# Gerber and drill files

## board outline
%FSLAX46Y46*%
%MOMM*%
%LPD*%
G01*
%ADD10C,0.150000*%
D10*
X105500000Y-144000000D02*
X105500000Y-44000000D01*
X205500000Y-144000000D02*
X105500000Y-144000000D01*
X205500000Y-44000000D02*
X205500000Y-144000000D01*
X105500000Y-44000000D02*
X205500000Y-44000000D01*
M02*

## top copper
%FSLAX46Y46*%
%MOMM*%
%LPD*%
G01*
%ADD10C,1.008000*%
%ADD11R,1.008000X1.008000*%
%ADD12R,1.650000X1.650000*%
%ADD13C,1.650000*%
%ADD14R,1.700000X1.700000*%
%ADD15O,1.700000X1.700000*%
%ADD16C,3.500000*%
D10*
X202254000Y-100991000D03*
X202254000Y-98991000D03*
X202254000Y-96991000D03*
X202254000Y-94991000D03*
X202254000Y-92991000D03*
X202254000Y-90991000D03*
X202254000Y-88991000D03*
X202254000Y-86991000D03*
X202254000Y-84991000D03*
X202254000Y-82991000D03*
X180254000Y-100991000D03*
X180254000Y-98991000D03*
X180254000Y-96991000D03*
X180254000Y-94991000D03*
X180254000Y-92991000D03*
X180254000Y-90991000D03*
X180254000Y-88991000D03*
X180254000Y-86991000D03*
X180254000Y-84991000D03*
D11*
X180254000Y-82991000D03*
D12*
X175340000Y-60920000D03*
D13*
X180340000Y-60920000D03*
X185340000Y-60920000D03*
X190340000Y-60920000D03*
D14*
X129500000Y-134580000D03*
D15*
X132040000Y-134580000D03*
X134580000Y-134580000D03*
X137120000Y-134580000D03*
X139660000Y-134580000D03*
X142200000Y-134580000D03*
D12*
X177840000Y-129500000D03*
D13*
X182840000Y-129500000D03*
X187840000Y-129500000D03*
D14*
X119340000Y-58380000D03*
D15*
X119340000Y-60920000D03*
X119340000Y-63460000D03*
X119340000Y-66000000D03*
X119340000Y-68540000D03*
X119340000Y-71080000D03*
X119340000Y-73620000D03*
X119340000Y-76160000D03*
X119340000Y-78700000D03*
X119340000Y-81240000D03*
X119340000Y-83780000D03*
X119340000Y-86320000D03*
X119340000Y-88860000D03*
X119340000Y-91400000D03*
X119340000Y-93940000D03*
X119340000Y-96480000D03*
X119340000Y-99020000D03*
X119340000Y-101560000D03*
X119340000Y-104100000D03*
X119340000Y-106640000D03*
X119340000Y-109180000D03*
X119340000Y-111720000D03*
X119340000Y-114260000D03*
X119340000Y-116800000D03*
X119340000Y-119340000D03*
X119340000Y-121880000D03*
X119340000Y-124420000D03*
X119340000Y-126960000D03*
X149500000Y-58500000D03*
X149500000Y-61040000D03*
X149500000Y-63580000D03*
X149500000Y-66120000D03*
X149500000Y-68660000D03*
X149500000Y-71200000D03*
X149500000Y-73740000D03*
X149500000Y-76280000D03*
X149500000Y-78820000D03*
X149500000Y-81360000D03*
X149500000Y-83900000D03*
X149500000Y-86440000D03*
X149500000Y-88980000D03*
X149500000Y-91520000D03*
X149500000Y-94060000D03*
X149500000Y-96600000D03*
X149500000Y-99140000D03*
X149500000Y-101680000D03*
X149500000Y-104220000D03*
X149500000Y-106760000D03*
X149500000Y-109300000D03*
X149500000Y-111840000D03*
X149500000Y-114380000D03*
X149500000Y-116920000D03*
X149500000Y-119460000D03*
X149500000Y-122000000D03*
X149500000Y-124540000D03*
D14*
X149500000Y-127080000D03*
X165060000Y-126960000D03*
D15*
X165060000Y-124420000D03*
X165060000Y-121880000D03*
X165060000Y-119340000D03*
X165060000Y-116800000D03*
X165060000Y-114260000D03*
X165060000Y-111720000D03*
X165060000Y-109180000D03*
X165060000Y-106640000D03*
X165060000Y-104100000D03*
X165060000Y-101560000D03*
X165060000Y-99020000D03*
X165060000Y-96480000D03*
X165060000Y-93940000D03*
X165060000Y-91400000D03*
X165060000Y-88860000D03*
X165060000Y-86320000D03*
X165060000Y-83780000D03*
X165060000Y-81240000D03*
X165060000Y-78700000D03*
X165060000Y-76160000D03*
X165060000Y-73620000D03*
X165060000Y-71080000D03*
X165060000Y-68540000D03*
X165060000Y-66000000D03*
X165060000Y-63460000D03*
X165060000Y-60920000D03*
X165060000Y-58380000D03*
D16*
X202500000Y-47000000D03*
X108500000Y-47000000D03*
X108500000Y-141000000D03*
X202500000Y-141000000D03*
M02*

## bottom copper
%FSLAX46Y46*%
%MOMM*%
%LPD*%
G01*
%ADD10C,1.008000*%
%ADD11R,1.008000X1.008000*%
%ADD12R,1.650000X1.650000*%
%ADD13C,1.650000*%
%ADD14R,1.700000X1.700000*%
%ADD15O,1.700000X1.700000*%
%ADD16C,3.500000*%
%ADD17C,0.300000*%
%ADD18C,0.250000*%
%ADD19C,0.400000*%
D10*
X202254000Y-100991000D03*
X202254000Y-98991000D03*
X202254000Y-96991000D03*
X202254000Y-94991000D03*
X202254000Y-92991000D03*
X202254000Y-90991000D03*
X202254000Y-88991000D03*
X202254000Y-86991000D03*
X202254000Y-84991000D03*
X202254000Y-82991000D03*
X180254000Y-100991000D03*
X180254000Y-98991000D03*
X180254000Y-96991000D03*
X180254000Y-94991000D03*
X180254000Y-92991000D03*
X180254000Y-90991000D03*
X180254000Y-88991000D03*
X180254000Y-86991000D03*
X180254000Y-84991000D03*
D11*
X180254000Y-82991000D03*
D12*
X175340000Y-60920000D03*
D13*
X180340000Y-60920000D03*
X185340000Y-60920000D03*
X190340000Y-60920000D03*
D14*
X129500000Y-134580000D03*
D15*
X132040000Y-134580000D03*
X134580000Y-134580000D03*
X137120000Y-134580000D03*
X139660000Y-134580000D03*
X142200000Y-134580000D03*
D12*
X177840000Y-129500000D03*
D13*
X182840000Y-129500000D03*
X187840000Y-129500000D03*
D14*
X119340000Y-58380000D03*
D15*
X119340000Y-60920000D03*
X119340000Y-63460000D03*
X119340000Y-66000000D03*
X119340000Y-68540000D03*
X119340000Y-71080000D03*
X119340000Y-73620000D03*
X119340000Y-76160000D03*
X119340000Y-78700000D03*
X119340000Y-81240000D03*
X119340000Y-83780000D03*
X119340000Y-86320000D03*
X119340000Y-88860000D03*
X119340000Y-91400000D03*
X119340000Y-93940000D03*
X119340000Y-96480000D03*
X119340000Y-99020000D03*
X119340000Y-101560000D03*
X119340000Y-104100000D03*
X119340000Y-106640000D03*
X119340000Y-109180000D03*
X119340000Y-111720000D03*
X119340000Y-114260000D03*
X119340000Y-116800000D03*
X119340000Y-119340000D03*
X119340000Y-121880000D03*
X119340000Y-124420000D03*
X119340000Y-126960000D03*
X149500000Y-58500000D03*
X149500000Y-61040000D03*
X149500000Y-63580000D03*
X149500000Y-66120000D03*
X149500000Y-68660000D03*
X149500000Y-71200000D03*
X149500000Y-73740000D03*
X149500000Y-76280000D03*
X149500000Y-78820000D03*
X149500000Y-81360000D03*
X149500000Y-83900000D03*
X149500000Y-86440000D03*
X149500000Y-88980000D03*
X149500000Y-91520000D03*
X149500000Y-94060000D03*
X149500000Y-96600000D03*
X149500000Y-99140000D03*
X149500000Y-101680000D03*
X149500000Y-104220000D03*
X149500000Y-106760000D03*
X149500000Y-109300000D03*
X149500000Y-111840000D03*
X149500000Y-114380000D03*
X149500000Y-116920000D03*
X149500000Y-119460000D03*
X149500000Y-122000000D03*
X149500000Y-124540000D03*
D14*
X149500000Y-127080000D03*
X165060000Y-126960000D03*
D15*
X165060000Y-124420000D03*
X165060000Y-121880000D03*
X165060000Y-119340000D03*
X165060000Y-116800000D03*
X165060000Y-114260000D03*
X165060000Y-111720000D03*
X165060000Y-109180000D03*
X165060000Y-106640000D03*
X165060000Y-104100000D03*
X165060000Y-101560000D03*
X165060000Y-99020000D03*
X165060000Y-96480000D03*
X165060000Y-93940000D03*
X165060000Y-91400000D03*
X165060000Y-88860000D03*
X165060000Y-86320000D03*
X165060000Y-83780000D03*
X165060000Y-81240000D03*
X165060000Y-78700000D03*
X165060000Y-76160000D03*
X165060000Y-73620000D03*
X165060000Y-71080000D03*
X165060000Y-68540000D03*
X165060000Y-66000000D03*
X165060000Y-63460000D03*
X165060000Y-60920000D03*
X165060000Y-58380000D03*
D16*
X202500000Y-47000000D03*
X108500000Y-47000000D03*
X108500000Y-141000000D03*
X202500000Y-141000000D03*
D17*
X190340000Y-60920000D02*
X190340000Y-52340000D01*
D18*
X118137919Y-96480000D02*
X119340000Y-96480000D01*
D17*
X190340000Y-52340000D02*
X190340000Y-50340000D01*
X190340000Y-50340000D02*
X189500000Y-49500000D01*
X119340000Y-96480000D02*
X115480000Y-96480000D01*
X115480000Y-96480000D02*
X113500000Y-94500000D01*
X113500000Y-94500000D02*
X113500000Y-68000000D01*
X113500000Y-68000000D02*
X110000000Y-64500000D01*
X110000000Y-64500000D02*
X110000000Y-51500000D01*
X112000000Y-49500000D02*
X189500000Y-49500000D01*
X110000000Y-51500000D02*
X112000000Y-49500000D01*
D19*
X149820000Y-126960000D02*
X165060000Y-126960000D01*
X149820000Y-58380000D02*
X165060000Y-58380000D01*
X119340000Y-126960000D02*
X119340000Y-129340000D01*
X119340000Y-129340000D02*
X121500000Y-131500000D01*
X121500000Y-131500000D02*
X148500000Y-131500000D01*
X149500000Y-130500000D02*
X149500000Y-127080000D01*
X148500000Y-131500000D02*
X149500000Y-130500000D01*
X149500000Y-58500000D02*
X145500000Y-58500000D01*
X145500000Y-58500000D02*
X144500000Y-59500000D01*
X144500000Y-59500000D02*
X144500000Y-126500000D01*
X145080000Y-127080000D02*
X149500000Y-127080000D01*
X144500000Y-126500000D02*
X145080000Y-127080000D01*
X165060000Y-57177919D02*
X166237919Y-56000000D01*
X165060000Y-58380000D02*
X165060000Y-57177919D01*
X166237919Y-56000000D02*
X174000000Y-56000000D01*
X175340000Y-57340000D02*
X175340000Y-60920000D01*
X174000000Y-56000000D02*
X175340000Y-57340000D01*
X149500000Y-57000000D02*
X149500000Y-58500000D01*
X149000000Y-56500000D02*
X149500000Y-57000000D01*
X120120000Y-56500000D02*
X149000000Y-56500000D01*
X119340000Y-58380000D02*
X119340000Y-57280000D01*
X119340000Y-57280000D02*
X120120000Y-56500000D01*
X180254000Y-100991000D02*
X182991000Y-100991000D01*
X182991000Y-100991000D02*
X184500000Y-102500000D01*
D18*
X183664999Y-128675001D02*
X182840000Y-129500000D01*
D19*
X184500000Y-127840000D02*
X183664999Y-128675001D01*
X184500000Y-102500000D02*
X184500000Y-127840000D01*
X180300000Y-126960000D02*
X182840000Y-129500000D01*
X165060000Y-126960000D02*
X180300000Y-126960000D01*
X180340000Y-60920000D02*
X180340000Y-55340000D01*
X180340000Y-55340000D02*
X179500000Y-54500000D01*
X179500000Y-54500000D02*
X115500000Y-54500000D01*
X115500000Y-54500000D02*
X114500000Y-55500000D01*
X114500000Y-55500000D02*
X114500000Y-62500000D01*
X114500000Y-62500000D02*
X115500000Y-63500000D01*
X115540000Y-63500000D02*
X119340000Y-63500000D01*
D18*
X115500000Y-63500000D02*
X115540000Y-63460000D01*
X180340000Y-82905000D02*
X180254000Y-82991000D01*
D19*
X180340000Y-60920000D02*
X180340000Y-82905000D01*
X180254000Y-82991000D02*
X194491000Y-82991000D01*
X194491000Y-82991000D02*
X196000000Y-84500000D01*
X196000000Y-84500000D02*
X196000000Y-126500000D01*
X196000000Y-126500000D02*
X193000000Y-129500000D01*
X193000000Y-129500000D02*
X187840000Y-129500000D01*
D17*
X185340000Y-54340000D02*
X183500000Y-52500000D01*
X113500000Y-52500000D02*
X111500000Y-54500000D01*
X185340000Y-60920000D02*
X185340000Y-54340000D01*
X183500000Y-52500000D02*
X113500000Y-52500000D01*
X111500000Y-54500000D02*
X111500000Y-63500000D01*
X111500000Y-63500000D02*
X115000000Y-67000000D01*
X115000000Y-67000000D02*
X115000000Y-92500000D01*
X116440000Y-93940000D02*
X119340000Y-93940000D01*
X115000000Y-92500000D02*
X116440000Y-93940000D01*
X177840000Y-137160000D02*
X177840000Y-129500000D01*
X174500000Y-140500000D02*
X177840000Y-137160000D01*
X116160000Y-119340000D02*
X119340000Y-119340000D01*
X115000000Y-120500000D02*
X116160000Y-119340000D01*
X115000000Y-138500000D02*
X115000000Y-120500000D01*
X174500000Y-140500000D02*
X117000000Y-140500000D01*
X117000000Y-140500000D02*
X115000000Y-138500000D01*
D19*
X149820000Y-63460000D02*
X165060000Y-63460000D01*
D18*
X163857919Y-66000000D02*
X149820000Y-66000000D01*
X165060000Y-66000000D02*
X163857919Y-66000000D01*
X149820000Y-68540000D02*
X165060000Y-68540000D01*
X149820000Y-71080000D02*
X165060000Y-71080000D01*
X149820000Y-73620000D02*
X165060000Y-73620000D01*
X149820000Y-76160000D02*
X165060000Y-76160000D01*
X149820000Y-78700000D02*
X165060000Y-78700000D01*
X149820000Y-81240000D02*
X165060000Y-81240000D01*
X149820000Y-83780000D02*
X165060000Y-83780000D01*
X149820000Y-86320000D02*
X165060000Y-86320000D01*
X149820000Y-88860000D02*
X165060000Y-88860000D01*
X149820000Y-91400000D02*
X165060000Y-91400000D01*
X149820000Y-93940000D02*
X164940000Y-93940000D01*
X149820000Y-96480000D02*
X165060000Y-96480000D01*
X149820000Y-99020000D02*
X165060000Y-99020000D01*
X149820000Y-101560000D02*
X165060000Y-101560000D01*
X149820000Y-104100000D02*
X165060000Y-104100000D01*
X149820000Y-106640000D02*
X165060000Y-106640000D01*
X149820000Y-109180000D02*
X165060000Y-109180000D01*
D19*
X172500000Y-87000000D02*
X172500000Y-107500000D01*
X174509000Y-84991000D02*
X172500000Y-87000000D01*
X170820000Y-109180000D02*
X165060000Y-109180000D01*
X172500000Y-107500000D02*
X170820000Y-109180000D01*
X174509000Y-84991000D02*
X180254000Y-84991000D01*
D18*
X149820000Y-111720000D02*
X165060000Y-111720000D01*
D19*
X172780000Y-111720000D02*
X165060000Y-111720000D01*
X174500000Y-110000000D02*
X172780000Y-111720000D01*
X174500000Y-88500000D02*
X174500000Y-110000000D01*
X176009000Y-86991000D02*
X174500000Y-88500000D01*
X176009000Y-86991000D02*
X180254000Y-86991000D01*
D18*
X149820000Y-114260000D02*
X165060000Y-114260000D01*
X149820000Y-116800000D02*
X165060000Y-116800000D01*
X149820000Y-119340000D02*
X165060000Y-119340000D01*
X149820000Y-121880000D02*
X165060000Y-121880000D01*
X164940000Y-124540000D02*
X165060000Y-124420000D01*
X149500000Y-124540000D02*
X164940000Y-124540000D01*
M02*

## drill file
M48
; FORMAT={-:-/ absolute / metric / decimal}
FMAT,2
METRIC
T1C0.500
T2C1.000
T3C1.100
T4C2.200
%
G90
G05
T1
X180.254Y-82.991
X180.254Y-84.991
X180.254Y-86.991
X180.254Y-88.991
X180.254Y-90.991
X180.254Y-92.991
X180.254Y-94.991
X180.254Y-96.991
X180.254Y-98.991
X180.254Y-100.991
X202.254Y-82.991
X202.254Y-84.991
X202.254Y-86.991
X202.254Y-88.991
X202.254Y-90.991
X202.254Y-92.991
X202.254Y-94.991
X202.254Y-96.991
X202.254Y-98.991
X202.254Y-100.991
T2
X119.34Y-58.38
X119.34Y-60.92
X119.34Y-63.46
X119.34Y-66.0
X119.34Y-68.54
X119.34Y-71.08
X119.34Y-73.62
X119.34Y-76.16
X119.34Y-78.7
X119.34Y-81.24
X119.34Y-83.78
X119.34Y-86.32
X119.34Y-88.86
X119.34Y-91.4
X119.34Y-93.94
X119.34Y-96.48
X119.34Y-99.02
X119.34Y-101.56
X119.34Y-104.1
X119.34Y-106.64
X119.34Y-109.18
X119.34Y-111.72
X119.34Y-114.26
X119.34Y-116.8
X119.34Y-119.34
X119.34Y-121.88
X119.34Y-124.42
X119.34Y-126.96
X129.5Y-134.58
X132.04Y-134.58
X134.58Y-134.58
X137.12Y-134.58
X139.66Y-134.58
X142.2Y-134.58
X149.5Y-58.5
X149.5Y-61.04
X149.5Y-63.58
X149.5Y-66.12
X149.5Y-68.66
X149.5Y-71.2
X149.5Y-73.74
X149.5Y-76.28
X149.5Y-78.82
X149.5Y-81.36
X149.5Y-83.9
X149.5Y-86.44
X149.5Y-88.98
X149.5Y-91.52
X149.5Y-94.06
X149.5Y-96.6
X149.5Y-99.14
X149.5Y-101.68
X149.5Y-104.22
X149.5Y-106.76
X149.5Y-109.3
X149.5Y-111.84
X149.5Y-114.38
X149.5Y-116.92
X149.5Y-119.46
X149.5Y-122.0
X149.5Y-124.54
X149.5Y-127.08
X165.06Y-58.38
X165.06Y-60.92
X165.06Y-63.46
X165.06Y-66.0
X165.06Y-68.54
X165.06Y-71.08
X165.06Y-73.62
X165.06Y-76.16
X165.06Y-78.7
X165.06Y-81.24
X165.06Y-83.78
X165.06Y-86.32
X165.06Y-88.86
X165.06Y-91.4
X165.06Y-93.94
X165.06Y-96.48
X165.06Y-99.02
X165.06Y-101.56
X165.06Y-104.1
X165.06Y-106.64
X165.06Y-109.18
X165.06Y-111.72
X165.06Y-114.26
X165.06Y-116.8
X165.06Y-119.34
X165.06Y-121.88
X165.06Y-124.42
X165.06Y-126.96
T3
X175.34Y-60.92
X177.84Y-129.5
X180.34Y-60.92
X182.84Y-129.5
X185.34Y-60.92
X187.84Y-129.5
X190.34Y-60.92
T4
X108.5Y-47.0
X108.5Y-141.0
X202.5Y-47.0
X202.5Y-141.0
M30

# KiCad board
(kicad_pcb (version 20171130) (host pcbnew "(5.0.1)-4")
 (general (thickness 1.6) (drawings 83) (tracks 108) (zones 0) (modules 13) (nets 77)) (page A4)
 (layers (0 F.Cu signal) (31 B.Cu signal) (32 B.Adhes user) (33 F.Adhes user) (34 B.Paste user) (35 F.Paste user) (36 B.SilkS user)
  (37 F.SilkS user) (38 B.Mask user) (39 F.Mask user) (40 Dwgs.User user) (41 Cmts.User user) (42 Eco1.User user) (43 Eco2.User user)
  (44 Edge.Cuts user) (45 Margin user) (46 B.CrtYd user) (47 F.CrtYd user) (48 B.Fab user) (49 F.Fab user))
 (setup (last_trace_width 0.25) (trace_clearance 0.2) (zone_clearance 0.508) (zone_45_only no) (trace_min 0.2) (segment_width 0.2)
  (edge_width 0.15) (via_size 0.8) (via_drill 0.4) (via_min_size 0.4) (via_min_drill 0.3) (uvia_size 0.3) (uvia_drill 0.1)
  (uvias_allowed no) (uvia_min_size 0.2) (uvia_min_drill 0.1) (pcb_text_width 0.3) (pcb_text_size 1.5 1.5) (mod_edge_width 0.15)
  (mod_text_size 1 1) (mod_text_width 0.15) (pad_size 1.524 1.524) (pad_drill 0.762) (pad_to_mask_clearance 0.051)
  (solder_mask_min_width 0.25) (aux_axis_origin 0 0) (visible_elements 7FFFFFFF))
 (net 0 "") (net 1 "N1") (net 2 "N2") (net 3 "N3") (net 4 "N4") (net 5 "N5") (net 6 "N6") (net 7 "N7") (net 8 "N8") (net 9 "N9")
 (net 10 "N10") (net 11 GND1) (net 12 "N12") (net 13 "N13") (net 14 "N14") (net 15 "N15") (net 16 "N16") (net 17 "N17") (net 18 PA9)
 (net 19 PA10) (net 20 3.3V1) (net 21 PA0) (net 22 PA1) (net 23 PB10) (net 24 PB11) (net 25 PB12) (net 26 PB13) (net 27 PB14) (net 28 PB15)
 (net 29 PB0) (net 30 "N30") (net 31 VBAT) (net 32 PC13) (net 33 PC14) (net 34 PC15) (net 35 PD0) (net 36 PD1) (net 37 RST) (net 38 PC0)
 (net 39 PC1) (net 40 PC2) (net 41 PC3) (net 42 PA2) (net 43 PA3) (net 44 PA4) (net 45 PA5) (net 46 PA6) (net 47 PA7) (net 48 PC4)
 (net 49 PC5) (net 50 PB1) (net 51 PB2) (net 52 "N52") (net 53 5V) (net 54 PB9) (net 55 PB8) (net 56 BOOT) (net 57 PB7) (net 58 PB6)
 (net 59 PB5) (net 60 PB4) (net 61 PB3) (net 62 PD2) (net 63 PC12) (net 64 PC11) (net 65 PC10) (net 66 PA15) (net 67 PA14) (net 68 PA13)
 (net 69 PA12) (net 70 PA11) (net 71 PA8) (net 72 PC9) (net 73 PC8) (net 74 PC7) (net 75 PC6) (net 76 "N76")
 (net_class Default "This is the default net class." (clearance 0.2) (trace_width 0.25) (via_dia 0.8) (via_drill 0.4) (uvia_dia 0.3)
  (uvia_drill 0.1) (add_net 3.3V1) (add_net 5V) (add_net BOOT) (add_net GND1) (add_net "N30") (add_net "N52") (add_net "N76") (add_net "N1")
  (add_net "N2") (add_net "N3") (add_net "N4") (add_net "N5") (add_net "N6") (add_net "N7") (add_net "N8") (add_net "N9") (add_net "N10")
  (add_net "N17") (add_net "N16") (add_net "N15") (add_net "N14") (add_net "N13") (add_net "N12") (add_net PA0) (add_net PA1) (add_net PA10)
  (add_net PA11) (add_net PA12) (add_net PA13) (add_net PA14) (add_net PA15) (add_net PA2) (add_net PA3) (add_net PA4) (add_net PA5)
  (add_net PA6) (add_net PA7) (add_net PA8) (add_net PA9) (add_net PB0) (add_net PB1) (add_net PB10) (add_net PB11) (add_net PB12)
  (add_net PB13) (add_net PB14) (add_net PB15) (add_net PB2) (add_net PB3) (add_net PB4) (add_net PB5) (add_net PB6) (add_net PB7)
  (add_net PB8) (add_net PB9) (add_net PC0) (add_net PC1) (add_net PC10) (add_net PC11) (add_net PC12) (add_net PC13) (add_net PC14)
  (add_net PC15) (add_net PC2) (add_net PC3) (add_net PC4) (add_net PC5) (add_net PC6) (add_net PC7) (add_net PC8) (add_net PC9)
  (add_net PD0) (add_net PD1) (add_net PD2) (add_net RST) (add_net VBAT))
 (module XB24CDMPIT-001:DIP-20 (layer F.Cu) (at 179 109)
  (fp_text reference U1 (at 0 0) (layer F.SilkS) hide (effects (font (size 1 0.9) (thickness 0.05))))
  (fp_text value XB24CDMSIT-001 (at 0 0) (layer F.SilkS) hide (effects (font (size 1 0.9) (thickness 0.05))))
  (pad 11 thru_hole circle (at 23.254 -8.009) (size 1.008 1.008) (drill 0.5) (layers *.Cu *.Mask) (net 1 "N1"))
  (pad 12 thru_hole circle (at 23.254 -10.009) (size 1.008 1.008) (drill 0.5) (layers *.Cu *.Mask) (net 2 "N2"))
  (pad 13 thru_hole circle (at 23.254 -12.009) (size 1.008 1.008) (drill 0.5) (layers *.Cu *.Mask) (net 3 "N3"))
  (pad 14 thru_hole circle (at 23.254 -14.009) (size 1.008 1.008) (drill 0.5) (layers *.Cu *.Mask) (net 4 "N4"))
  (pad 15 thru_hole circle (at 23.254 -16.009) (size 1.008 1.008) (drill 0.5) (layers *.Cu *.Mask) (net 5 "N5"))
  (pad 16 thru_hole circle (at 23.254 -18.009) (size 1.008 1.008) (drill 0.5) (layers *.Cu *.Mask) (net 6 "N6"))
  (pad 17 thru_hole circle (at 23.254 -20.009) (size 1.008 1.008) (drill 0.5) (layers *.Cu *.Mask) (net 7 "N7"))
  (pad 18 thru_hole circle (at 23.254 -22.009) (size 1.008 1.008) (drill 0.5) (layers *.Cu *.Mask) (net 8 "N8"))
  (pad 19 thru_hole circle (at 23.254 -24.009) (size 1.008 1.008) (drill 0.5) (layers *.Cu *.Mask) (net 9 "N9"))
  (pad 20 thru_hole circle (at 23.254 -26.009) (size 1.008 1.008) (drill 0.5) (layers *.Cu *.Mask) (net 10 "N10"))
  (pad 10 thru_hole circle (at 1.254 -8.009) (size 1.008 1.008) (drill 0.5) (layers *.Cu *.Mask) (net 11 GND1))
  (pad 9 thru_hole circle (at 1.254 -10.009) (size 1.008 1.008) (drill 0.5) (layers *.Cu *.Mask) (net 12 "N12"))
  (pad 8 thru_hole circle (at 1.254 -12.009) (size 1.008 1.008) (drill 0.5) (layers *.Cu *.Mask) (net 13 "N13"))
  (pad 7 thru_hole circle (at 1.254 -14.009) (size 1.008 1.008) (drill 0.5) (layers *.Cu *.Mask) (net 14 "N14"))
  (pad 6 thru_hole circle (at 1.254 -16.009) (size 1.008 1.008) (drill 0.5) (layers *.Cu *.Mask) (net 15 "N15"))
  (pad 5 thru_hole circle (at 1.254 -18.009) (size 1.008 1.008) (drill 0.5) (layers *.Cu *.Mask) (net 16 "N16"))
  (pad 4 thru_hole circle (at 1.254 -20.009) (size 1.008 1.008) (drill 0.5) (layers *.Cu *.Mask) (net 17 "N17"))
  (pad 3 thru_hole circle (at 1.254 -22.009) (size 1.008 1.008) (drill 0.5) (layers *.Cu *.Mask) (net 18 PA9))
  (pad 2 thru_hole circle (at 1.254 -24.009) (size 1.008 1.008) (drill 0.5) (layers *.Cu *.Mask) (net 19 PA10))
  (pad 1 thru_hole rect (at 1.254 -26.009) (size 1.008 1.008) (drill 0.5) (layers *.Cu *.Mask) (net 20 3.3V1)))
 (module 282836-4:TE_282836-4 (layer F.Cu) (at 182.84 60.92)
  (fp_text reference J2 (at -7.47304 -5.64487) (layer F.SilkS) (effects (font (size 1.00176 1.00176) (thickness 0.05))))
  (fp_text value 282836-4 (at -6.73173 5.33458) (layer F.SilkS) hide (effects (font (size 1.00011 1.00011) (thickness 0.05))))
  (pad 1 thru_hole rect (at -7.5 0) (size 1.65 1.65) (drill 1.1) (layers *.Cu *.Mask) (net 11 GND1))
  (pad 2 thru_hole circle (at -2.5 0) (size 1.65 1.65) (drill 1.1) (layers *.Cu *.Mask) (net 20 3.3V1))
  (pad 3 thru_hole circle (at 2.5 0) (size 1.65 1.65) (drill 1.1) (layers *.Cu *.Mask) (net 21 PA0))
  (pad 4 thru_hole circle (at 7.5 0) (size 1.65 1.65) (drill 1.1) (layers *.Cu *.Mask) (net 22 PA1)))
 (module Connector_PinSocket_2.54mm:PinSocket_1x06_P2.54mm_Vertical (layer F.Cu) (at 129.5 134.58 90)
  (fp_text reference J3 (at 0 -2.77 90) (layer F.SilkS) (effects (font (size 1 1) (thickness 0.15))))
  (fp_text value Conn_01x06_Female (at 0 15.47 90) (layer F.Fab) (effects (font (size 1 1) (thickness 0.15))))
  (pad 1 thru_hole rect (at 0 0 90) (size 1.7 1.7) (drill 1) (layers *.Cu *.Mask) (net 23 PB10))
  (pad 2 thru_hole oval (at 0 2.54 90) (size 1.7 1.7) (drill 1) (layers *.Cu *.Mask) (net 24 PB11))
  (pad 3 thru_hole oval (at 0 5.08 90) (size 1.7 1.7) (drill 1) (layers *.Cu *.Mask) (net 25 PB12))
  (pad 4 thru_hole oval (at 0 7.62 90) (size 1.7 1.7) (drill 1) (layers *.Cu *.Mask) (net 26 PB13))
  (pad 5 thru_hole oval (at 0 10.16 90) (size 1.7 1.7) (drill 1) (layers *.Cu *.Mask) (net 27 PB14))
  (pad 6 thru_hole oval (at 0 12.7 90) (size 1.7 1.7) (drill 1) (layers *.Cu *.Mask) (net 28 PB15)))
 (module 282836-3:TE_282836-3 (layer F.Cu) (at 182.84 129.5)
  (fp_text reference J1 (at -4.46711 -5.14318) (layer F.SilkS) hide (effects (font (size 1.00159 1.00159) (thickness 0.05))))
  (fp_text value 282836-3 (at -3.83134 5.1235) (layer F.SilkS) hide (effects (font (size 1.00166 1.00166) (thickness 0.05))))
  (pad 1 thru_hole rect (at -5 0) (size 1.65 1.65) (drill 1.1) (layers *.Cu *.Mask) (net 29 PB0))
  (pad 2 thru_hole circle (at 0 0) (size 1.65 1.65) (drill 1.1) (layers *.Cu *.Mask) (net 11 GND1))
  (pad 3 thru_hole circle (at 5 0) (size 1.65 1.65) (drill 1.1) (layers *.Cu *.Mask) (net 20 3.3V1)))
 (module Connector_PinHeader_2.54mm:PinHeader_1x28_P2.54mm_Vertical (layer F.Cu) (at 119.34 58.38)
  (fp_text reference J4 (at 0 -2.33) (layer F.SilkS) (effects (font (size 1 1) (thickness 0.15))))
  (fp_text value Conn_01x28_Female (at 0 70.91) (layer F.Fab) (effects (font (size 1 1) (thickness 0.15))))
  (pad 1 thru_hole rect (at 0 0) (size 1.7 1.7) (drill 1) (layers *.Cu *.Mask) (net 11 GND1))
  (pad 2 thru_hole oval (at 0 2.54) (size 1.7 1.7) (drill 1) (layers *.Cu *.Mask) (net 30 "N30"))
  (pad 3 thru_hole oval (at 0 5.08) (size 1.7 1.7) (drill 1) (layers *.Cu *.Mask) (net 20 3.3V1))
  (pad 4 thru_hole oval (at 0 7.62) (size 1.7 1.7) (drill 1) (layers *.Cu *.Mask) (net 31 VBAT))
  (pad 5 thru_hole oval (at 0 10.16) (size 1.7 1.7) (drill 1) (layers *.Cu *.Mask) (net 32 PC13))
  (pad 6 thru_hole oval (at 0 12.7) (size 1.7 1.7) (drill 1) (layers *.Cu *.Mask) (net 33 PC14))
  (pad 7 thru_hole oval (at 0 15.24) (size 1.7 1.7) (drill 1) (layers *.Cu *.Mask) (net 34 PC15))
  (pad 8 thru_hole oval (at 0 17.78) (size 1.7 1.7) (drill 1) (layers *.Cu *.Mask) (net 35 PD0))
  (pad 9 thru_hole oval (at 0 20.32) (size 1.7 1.7) (drill 1) (layers *.Cu *.Mask) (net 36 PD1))
  (pad 10 thru_hole oval (at 0 22.86) (size 1.7 1.7) (drill 1) (layers *.Cu *.Mask) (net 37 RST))
  (pad 11 thru_hole oval (at 0 25.4) (size 1.7 1.7) (drill 1) (layers *.Cu *.Mask) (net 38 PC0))
  (pad 12 thru_hole oval (at 0 27.94) (size 1.7 1.7) (drill 1) (layers *.Cu *.Mask) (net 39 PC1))
  (pad 13 thru_hole oval (at 0 30.48) (size 1.7 1.7) (drill 1) (layers *.Cu *.Mask) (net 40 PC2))
  (pad 14 thru_hole oval (at 0 33.02) (size 1.7 1.7) (drill 1) (layers *.Cu *.Mask) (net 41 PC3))
  (pad 15 thru_hole oval (at 0 35.56) (size 1.7 1.7) (drill 1) (layers *.Cu *.Mask) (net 21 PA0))
  (pad 16 thru_hole oval (at 0 38.1) (size 1.7 1.7) (drill 1) (layers *.Cu *.Mask) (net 22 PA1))
  (pad 17 thru_hole oval (at 0 40.64) (size 1.7 1.7) (drill 1) (layers *.Cu *.Mask) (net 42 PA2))
  (pad 18 thru_hole oval (at 0 43.18) (size 1.7 1.7) (drill 1) (layers *.Cu *.Mask) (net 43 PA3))
  (pad 19 thru_hole oval (at 0 45.72) (size 1.7 1.7) (drill 1) (layers *.Cu *.Mask) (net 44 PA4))
  (pad 20 thru_hole oval (at 0 48.26) (size 1.7 1.7) (drill 1) (layers *.Cu *.Mask) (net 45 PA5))
  (pad 21 thru_hole oval (at 0 50.8) (size 1.7 1.7) (drill 1) (layers *.Cu *.Mask) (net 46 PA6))
  (pad 22 thru_hole oval (at 0 53.34) (size 1.7 1.7) (drill 1) (layers *.Cu *.Mask) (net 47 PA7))
  (pad 23 thru_hole oval (at 0 55.88) (size 1.7 1.7) (drill 1) (layers *.Cu *.Mask) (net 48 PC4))
  (pad 24 thru_hole oval (at 0 58.42) (size 1.7 1.7) (drill 1) (layers *.Cu *.Mask) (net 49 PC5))
  (pad 25 thru_hole oval (at 0 60.96) (size 1.7 1.7) (drill 1) (layers *.Cu *.Mask) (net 29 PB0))
  (pad 26 thru_hole oval (at 0 63.5) (size 1.7 1.7) (drill 1) (layers *.Cu *.Mask) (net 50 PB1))
  (pad 27 thru_hole oval (at 0 66.04) (size 1.7 1.7) (drill 1) (layers *.Cu *.Mask) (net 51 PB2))
  (pad 28 thru_hole oval (at 0 68.58) (size 1.7 1.7) (drill 1) (layers *.Cu *.Mask) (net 11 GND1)))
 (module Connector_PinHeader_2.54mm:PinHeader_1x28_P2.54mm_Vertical (layer B.Cu) (at 149.5 127.08)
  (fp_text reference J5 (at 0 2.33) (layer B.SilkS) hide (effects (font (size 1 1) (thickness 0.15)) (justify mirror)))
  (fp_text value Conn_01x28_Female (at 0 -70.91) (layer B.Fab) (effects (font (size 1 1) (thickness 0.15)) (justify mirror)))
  (pad 28 thru_hole oval (at 0 -68.58) (size 1.7 1.7) (drill 1) (layers *.Cu *.Mask) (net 11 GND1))
  (pad 27 thru_hole oval (at 0 -66.04) (size 1.7 1.7) (drill 1) (layers *.Cu *.Mask) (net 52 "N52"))
  (pad 26 thru_hole oval (at 0 -63.5) (size 1.7 1.7) (drill 1) (layers *.Cu *.Mask) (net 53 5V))
  (pad 25 thru_hole oval (at 0 -60.96) (size 1.7 1.7) (drill 1) (layers *.Cu *.Mask) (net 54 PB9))
  (pad 24 thru_hole oval (at 0 -58.42) (size 1.7 1.7) (drill 1) (layers *.Cu *.Mask) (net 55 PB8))
  (pad 23 thru_hole oval (at 0 -55.88) (size 1.7 1.7) (drill 1) (layers *.Cu *.Mask) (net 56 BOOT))
  (pad 22 thru_hole oval (at 0 -53.34) (size 1.7 1.7) (drill 1) (layers *.Cu *.Mask) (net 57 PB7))
  (pad 21 thru_hole oval (at 0 -50.8) (size 1.7 1.7) (drill 1) (layers *.Cu *.Mask) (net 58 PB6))
  (pad 20 thru_hole oval (at 0 -48.26) (size 1.7 1.7) (drill 1) (layers *.Cu *.Mask) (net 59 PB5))
  (pad 19 thru_hole oval (at 0 -45.72) (size 1.7 1.7) (drill 1) (layers *.Cu *.Mask) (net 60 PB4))
  (pad 18 thru_hole oval (at 0 -43.18) (size 1.7 1.7) (drill 1) (layers *.Cu *.Mask) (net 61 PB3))
  (pad 17 thru_hole oval (at 0 -40.64) (size 1.7 1.7) (drill 1) (layers *.Cu *.Mask) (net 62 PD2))
  (pad 16 thru_hole oval (at 0 -38.1) (size 1.7 1.7) (drill 1) (layers *.Cu *.Mask) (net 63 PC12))
  (pad 15 thru_hole oval (at 0 -35.56) (size 1.7 1.7) (drill 1) (layers *.Cu *.Mask) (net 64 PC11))
  (pad 14 thru_hole oval (at 0 -33.02) (size 1.7 1.7) (drill 1) (layers *.Cu *.Mask) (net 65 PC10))
  (pad 13 thru_hole oval (at 0 -30.48) (size 1.7 1.7) (drill 1) (layers *.Cu *.Mask) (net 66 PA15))
  (pad 12 thru_hole oval (at 0 -27.94) (size 1.7 1.7) (drill 1) (layers *.Cu *.Mask) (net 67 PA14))
  (pad 11 thru_hole oval (at 0 -25.4) (size 1.7 1.7) (drill 1) (layers *.Cu *.Mask) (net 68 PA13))
  (pad 10 thru_hole oval (at 0 -22.86) (size 1.7 1.7) (drill 1) (layers *.Cu *.Mask) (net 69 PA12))
  (pad 9 thru_hole oval (at 0 -20.32) (size 1.7 1.7) (drill 1) (layers *.Cu *.Mask) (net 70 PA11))
  (pad 8 thru_hole oval (at 0 -17.78) (size 1.7 1.7) (drill 1) (layers *.Cu *.Mask) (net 19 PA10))
  (pad 7 thru_hole oval (at 0 -15.24) (size 1.7 1.7) (drill 1) (layers *.Cu *.Mask) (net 18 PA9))
  (pad 6 thru_hole oval (at 0 -12.7) (size 1.7 1.7) (drill 1) (layers *.Cu *.Mask) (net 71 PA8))
  (pad 5 thru_hole oval (at 0 -10.16) (size 1.7 1.7) (drill 1) (layers *.Cu *.Mask) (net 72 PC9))
  (pad 4 thru_hole oval (at 0 -7.62) (size 1.7 1.7) (drill 1) (layers *.Cu *.Mask) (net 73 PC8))
  (pad 3 thru_hole oval (at 0 -5.08) (size 1.7 1.7) (drill 1) (layers *.Cu *.Mask) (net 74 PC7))
  (pad 2 thru_hole oval (at 0 -2.54) (size 1.7 1.7) (drill 1) (layers *.Cu *.Mask) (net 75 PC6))
  (pad 1 thru_hole rect (at 0 0) (size 1.7 1.7) (drill 1) (layers *.Cu *.Mask) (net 11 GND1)))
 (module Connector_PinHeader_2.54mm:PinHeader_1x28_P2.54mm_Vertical (layer B.Cu) (at 165.06 126.96)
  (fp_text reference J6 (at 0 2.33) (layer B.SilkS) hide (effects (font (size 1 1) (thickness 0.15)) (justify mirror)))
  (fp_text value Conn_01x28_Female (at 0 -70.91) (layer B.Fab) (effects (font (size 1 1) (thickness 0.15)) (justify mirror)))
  (pad 1 thru_hole rect (at 0 0) (size 1.7 1.7) (drill 1) (layers *.Cu *.Mask) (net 11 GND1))
  (pad 2 thru_hole oval (at 0 -2.54) (size 1.7 1.7) (drill 1) (layers *.Cu *.Mask) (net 75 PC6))
  (pad 3 thru_hole oval (at 0 -5.08) (size 1.7 1.7) (drill 1) (layers *.Cu *.Mask) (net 74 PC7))
  (pad 4 thru_hole oval (at 0 -7.62) (size 1.7 1.7) (drill 1) (layers *.Cu *.Mask) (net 73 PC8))
  (pad 5 thru_hole oval (at 0 -10.16) (size 1.7 1.7) (drill 1) (layers *.Cu *.Mask) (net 72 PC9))
  (pad 6 thru_hole oval (at 0 -12.7) (size 1.7 1.7) (drill 1) (layers *.Cu *.Mask) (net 71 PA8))
  (pad 7 thru_hole oval (at 0 -15.24) (size 1.7 1.7) (drill 1) (layers *.Cu *.Mask) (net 18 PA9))
  (pad 8 thru_hole oval (at 0 -17.78) (size 1.7 1.7) (drill 1) (layers *.Cu *.Mask) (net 19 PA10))
  (pad 9 thru_hole oval (at 0 -20.32) (size 1.7 1.7) (drill 1) (layers *.Cu *.Mask) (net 70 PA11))
  (pad 10 thru_hole oval (at 0 -22.86) (size 1.7 1.7) (drill 1) (layers *.Cu *.Mask) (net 69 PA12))
  (pad 11 thru_hole oval (at 0 -25.4) (size 1.7 1.7) (drill 1) (layers *.Cu *.Mask) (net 68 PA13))
  (pad 12 thru_hole oval (at 0 -27.94) (size 1.7 1.7) (drill 1) (layers *.Cu *.Mask) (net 67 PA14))
  (pad 13 thru_hole oval (at 0 -30.48) (size 1.7 1.7) (drill 1) (layers *.Cu *.Mask) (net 66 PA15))
  (pad 14 thru_hole oval (at 0 -33.02) (size 1.7 1.7) (drill 1) (layers *.Cu *.Mask) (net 65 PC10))
  (pad 15 thru_hole oval (at 0 -35.56) (size 1.7 1.7) (drill 1) (layers *.Cu *.Mask) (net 64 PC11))
  (pad 16 thru_hole oval (at 0 -38.1) (size 1.7 1.7) (drill 1) (layers *.Cu *.Mask) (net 63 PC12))
  (pad 17 thru_hole oval (at 0 -40.64) (size 1.7 1.7) (drill 1) (layers *.Cu *.Mask) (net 62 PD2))
  (pad 18 thru_hole oval (at 0 -43.18) (size 1.7 1.7) (drill 1) (layers *.Cu *.Mask) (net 61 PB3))
  (pad 19 thru_hole oval (at 0 -45.72) (size 1.7 1.7) (drill 1) (layers *.Cu *.Mask) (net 60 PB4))
  (pad 20 thru_hole oval (at 0 -48.26) (size 1.7 1.7) (drill 1) (layers *.Cu *.Mask) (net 59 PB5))
  (pad 21 thru_hole oval (at 0 -50.8) (size 1.7 1.7) (drill 1) (layers *.Cu *.Mask) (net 58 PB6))
  (pad 22 thru_hole oval (at 0 -53.34) (size 1.7 1.7) (drill 1) (layers *.Cu *.Mask) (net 57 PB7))
  (pad 23 thru_hole oval (at 0 -55.88) (size 1.7 1.7) (drill 1) (layers *.Cu *.Mask) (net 56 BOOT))
  (pad 24 thru_hole oval (at 0 -58.42) (size 1.7 1.7) (drill 1) (layers *.Cu *.Mask) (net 55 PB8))
  (pad 25 thru_hole oval (at 0 -60.96) (size 1.7 1.7) (drill 1) (layers *.Cu *.Mask) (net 54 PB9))
  (pad 26 thru_hole oval (at 0 -63.5) (size 1.7 1.7) (drill 1) (layers *.Cu *.Mask) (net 53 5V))
  (pad 27 thru_hole oval (at 0 -66.04) (size 1.7 1.7) (drill 1) (layers *.Cu *.Mask) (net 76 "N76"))
  (pad 28 thru_hole oval (at 0 -68.58) (size 1.7 1.7) (drill 1) (layers *.Cu *.Mask) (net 11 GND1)))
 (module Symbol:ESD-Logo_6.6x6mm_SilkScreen (layer F.Cu) (at 191.5 113.5)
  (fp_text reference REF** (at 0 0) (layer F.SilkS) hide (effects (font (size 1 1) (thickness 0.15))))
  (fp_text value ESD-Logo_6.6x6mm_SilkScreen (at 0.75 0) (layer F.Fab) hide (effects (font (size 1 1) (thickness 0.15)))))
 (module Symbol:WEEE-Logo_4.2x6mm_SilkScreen (layer F.Cu) (at 201.5 61.5)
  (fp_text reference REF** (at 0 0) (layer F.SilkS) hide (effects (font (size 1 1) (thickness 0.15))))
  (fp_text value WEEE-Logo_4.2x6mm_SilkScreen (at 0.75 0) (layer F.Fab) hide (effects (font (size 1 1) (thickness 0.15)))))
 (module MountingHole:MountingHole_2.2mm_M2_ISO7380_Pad (layer F.Cu) (at 202.5 47)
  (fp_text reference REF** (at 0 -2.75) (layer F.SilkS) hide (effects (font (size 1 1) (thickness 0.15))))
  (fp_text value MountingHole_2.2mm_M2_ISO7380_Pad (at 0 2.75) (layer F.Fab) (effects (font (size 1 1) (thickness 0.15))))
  (pad 1 thru_hole circle (at 0 0) (size 3.5 3.5) (drill 2.2) (layers *.Cu *.Mask)))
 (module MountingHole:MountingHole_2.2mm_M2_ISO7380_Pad (layer F.Cu) (at 108.5 47)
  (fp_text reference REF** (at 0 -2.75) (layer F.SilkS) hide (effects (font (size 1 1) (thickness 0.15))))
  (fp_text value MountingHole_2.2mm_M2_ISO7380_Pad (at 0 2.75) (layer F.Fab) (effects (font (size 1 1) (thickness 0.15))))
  (pad 1 thru_hole circle (at 0 0) (size 3.5 3.5) (drill 2.2) (layers *.Cu *.Mask)))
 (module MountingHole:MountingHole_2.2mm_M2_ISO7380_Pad (layer F.Cu) (at 108.5 141)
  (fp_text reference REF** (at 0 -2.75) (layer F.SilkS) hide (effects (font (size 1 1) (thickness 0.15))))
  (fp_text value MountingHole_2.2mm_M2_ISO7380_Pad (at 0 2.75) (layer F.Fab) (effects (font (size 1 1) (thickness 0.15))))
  (pad 1 thru_hole circle (at 0 0) (size 3.5 3.5) (drill 2.2) (layers *.Cu *.Mask)))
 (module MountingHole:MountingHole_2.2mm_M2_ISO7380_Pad (layer F.Cu) (at 202.5 141)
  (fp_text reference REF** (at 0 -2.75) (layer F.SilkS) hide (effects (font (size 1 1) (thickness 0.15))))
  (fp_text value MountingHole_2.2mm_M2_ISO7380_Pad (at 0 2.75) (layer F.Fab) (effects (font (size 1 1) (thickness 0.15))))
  (pad 1 thru_hole circle (at 0 0) (size 3.5 3.5) (drill 2.2) (layers *.Cu *.Mask)))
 (gr_line (start 105.5 144) (end 105.5 44) (layer Edge.Cuts) (width 0.15))
 (gr_line (start 205.5 144) (end 105.5 144) (layer Edge.Cuts) (width 0.15))
 (gr_line (start 205.5 44) (end 205.5 144) (layer Edge.Cuts) (width 0.15))
 (gr_line (start 105.5 44) (end 205.5 44) (layer Edge.Cuts) (width 0.15))
 (segment (start 190.34 60.92) (end 190.34 52.34) (width 0.3) (layer B.Cu) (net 22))
 (segment (start 118.137919 96.48) (end 119.34 96.48) (width 0.25) (layer B.Cu) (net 22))
 (segment (start 190.34 52.34) (end 190.34 50.34) (width 0.3) (layer B.Cu) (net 22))
 (segment (start 190.34 50.34) (end 189.5 49.5) (width 0.3) (layer B.Cu) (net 22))
 (segment (start 119.34 96.48) (end 115.48 96.48) (width 0.3) (layer B.Cu) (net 22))
 (segment (start 115.48 96.48) (end 113.5 94.5) (width 0.3) (layer B.Cu) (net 22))
 (segment (start 113.5 94.5) (end 113.5 68) (width 0.3) (layer B.Cu) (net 22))
 (segment (start 113.5 68) (end 110 64.5) (width 0.3) (layer B.Cu) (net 22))
 (segment (start 110 64.5) (end 110 51.5) (width 0.3) (layer B.Cu) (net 22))
 (segment (start 112 49.5) (end 189.5 49.5) (width 0.3) (layer B.Cu) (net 22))
 (segment (start 110 51.5) (end 112 49.5) (width 0.3) (layer B.Cu) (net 22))
 (segment (start 149.82 126.96) (end 165.06 126.96) (width 0.4) (layer B.Cu) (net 11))
 (segment (start 149.82 58.38) (end 165.06 58.38) (width 0.4) (layer B.Cu) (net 11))
 (segment (start 119.34 126.96) (end 119.34 129.34) (width 0.4) (layer B.Cu) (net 11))
 (segment (start 119.34 129.34) (end 121.5 131.5) (width 0.4) (layer B.Cu) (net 11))
 (segment (start 121.5 131.5) (end 148.5 131.5) (width 0.4) (layer B.Cu) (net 11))
 (segment (start 149.5 130.5) (end 149.5 127.08) (width 0.4) (layer B.Cu) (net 11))
 (segment (start 148.5 131.5) (end 149.5 130.5) (width 0.4) (layer B.Cu) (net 11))
 (segment (start 149.5 58.5) (end 145.5 58.5) (width 0.4) (layer B.Cu) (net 11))
 (segment (start 145.5 58.5) (end 144.5 59.5) (width 0.4) (layer B.Cu) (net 11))
 (segment (start 144.5 59.5) (end 144.5 126.5) (width 0.4) (layer B.Cu) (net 11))
 (segment (start 145.08 127.08) (end 149.5 127.08) (width 0.4) (layer B.Cu) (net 11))
 (segment (start 144.5 126.5) (end 145.08 127.08) (width 0.4) (layer B.Cu) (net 11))
 (segment (start 165.06 57.177919) (end 166.237919 56) (width 0.4) (layer B.Cu) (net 11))
 (segment (start 165.06 58.38) (end 165.06 57.177919) (width 0.4) (layer B.Cu) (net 11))
 (segment (start 166.237919 56) (end 174 56) (width 0.4) (layer B.Cu) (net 11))
 (segment (start 175.34 57.34) (end 175.34 60.92) (width 0.4) (layer B.Cu) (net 11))
 (segment (start 174 56) (end 175.34 57.34) (width 0.4) (layer B.Cu) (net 11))
 (segment (start 149.5 57) (end 149.5 58.5) (width 0.4) (layer B.Cu) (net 11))
 (segment (start 149 56.5) (end 149.5 57) (width 0.4) (layer B.Cu) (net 11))
 (segment (start 120.12 56.5) (end 149 56.5) (width 0.4) (layer B.Cu) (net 11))
 (segment (start 119.34 58.38) (end 119.34 57.28) (width 0.4) (layer B.Cu) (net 11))
 (segment (start 119.34 57.28) (end 120.12 56.5) (width 0.4) (layer B.Cu) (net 11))
 (segment (start 180.254 100.991) (end 182.991 100.991) (width 0.4) (layer B.Cu) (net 11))
 (segment (start 182.991 100.991) (end 184.5 102.5) (width 0.4) (layer B.Cu) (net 11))
 (segment (start 183.664999 128.675001) (end 182.84 129.5) (width 0.25) (layer B.Cu) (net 11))
 (segment (start 184.5 127.84) (end 183.664999 128.675001) (width 0.4) (layer B.Cu) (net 11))
 (segment (start 184.5 102.5) (end 184.5 127.84) (width 0.4) (layer B.Cu) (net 11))
 (segment (start 180.3 126.96) (end 182.84 129.5) (width 0.4) (layer B.Cu) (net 11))
 (segment (start 165.06 126.96) (end 180.3 126.96) (width 0.4) (layer B.Cu) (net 11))
 (segment (start 180.34 60.92) (end 180.34 55.34) (width 0.4) (layer B.Cu) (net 20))
 (segment (start 180.34 55.34) (end 179.5 54.5) (width 0.4) (layer B.Cu) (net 20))
 (segment (start 179.5 54.5) (end 115.5 54.5) (width 0.4) (layer B.Cu) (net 20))
 (segment (start 115.5 54.5) (end 114.5 55.5) (width 0.4) (layer B.Cu) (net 20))
 (segment (start 114.5 55.5) (end 114.5 62.5) (width 0.4) (layer B.Cu) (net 20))
 (segment (start 114.5 62.5) (end 115.5 63.5) (width 0.4) (layer B.Cu) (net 20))
 (segment (start 115.54 63.5) (end 119.34 63.5) (width 0.4) (layer B.Cu) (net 20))
 (segment (start 115.5 63.5) (end 115.54 63.46) (width 0.25) (layer B.Cu) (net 20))
 (segment (start 180.34 82.905) (end 180.254 82.991) (width 0.25) (layer B.Cu) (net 20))
 (segment (start 180.34 60.92) (end 180.34 82.905) (width 0.4) (layer B.Cu) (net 20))
 (segment (start 180.254 82.991) (end 194.491 82.991) (width 0.4) (layer B.Cu) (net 20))
 (segment (start 194.491 82.991) (end 196 84.5) (width 0.4) (layer B.Cu) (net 20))
 (segment (start 196 84.5) (end 196 126.5) (width 0.4) (layer B.Cu) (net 20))
 (segment (start 196 126.5) (end 193 129.5) (width 0.4) (layer B.Cu) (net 20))
 (segment (start 193 129.5) (end 187.84 129.5) (width 0.4) (layer B.Cu) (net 20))
 (segment (start 185.34 54.34) (end 183.5 52.5) (width 0.3) (layer B.Cu) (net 21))
 (segment (start 113.5 52.5) (end 111.5 54.5) (width 0.3) (layer B.Cu) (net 21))
 (segment (start 185.34 60.92) (end 185.34 54.34) (width 0.3) (layer B.Cu) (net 21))
 (segment (start 183.5 52.5) (end 113.5 52.5) (width 0.3) (layer B.Cu) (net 21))
 (segment (start 111.5 54.5) (end 111.5 63.5) (width 0.3) (layer B.Cu) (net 21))
 (segment (start 111.5 63.5) (end 115 67) (width 0.3) (layer B.Cu) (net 21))
 (segment (start 115 67) (end 115 92.5) (width 0.3) (layer B.Cu) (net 21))
 (segment (start 116.44 93.94) (end 119.34 93.94) (width 0.3) (layer B.Cu) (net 21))
 (segment (start 115 92.5) (end 116.44 93.94) (width 0.3) (layer B.Cu) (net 21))
 (segment (start 177.84 137.16) (end 177.84 129.5) (width 0.3) (layer B.Cu) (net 29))
 (segment (start 174.5 140.5) (end 177.84 137.16) (width 0.3) (layer B.Cu) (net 29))
 (segment (start 116.16 119.34) (end 119.34 119.34) (width 0.3) (layer B.Cu) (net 29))
 (segment (start 115 120.5) (end 116.16 119.34) (width 0.3) (layer B.Cu) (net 29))
 (segment (start 115 138.5) (end 115 120.5) (width 0.3) (layer B.Cu) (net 29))
 (segment (start 174.5 140.5) (end 117 140.5) (width 0.3) (layer B.Cu) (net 29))
 (segment (start 117 140.5) (end 115 138.5) (width 0.3) (layer B.Cu) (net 29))
 (segment (start 149.82 63.46) (end 165.06 63.46) (width 0.4) (layer B.Cu) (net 53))
 (segment (start 163.857919 66) (end 149.82 66) (width 0.25) (layer B.Cu) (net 54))
 (segment (start 165.06 66) (end 163.857919 66) (width 0.25) (layer B.Cu) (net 54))
 (segment (start 149.82 68.54) (end 165.06 68.54) (width 0.25) (layer B.Cu) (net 55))
 (segment (start 149.82 71.08) (end 165.06 71.08) (width 0.25) (layer B.Cu) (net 56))
 (segment (start 149.82 73.62) (end 165.06 73.62) (width 0.25) (layer B.Cu) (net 57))
 (segment (start 149.82 76.16) (end 165.06 76.16) (width 0.25) (layer B.Cu) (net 58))
 (segment (start 149.82 78.7) (end 165.06 78.7) (width 0.25) (layer B.Cu) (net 59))
 (segment (start 149.82 81.24) (end 165.06 81.24) (width 0.25) (layer B.Cu) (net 60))
 (segment (start 149.82 83.78) (end 165.06 83.78) (width 0.25) (layer B.Cu) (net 61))
 (segment (start 149.82 86.32) (end 165.06 86.32) (width 0.25) (layer B.Cu) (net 62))
 (segment (start 149.82 88.86) (end 165.06 88.86) (width 0.25) (layer B.Cu) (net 63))
 (segment (start 149.82 91.4) (end 165.06 91.4) (width 0.25) (layer B.Cu) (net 64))
 (segment (start 149.82 93.94) (end 164.94 93.94) (width 0.25) (layer B.Cu) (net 65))
 (segment (start 149.82 96.48) (end 165.06 96.48) (width 0.25) (layer B.Cu) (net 66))
 (segment (start 149.82 99.02) (end 165.06 99.02) (width 0.25) (layer B.Cu) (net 67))
 (segment (start 149.82 101.56) (end 165.06 101.56) (width 0.25) (layer B.Cu) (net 68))
 (segment (start 149.82 104.1) (end 165.06 104.1) (width 0.25) (layer B.Cu) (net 69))
 (segment (start 149.82 106.64) (end 165.06 106.64) (width 0.25) (layer B.Cu) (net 70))
 (segment (start 149.82 109.18) (end 165.06 109.18) (width 0.25) (layer B.Cu) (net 19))
 (segment (start 172.5 87) (end 172.5 107.5) (width 0.4) (layer B.Cu) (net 19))
 (segment (start 174.509 84.991) (end 172.5 87) (width 0.4) (layer B.Cu) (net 19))
 (segment (start 170.82 109.18) (end 165.06 109.18) (width 0.4) (layer B.Cu) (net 19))
 (segment (start 172.5 107.5) (end 170.82 109.18) (width 0.4) (layer B.Cu) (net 19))
 (segment (start 174.509 84.991) (end 180.254 84.991) (width 0.4) (layer B.Cu) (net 19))
 (segment (start 149.82 111.72) (end 165.06 111.72) (width 0.25) (layer B.Cu) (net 18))
 (segment (start 172.78 111.72) (end 165.06 111.72) (width 0.4) (layer B.Cu) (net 18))
 (segment (start 174.5 110) (end 172.78 111.72) (width 0.4) (layer B.Cu) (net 18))
 (segment (start 174.5 88.5) (end 174.5 110) (width 0.4) (layer B.Cu) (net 18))
 (segment (start 176.009 86.991) (end 174.5 88.5) (width 0.4) (layer B.Cu) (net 18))
 (segment (start 176.009 86.991) (end 180.254 86.991) (width 0.4) (layer B.Cu) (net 18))
 (segment (start 149.82 114.26) (end 165.06 114.26) (width 0.25) (layer B.Cu) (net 71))
 (segment (start 149.82 116.8) (end 165.06 116.8) (width 0.25) (layer B.Cu) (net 72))
 (segment (start 149.82 119.34) (end 165.06 119.34) (width 0.25) (layer B.Cu) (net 73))
 (segment (start 149.82 121.88) (end 165.06 121.88) (width 0.25) (layer B.Cu) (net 74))
 (segment (start 164.94 124.54) (end 165.06 124.42) (width 0.25) (layer B.Cu) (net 75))
 (segment (start 149.5 124.54) (end 164.94 124.54) (width 0.25) (layer B.Cu) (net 75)))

